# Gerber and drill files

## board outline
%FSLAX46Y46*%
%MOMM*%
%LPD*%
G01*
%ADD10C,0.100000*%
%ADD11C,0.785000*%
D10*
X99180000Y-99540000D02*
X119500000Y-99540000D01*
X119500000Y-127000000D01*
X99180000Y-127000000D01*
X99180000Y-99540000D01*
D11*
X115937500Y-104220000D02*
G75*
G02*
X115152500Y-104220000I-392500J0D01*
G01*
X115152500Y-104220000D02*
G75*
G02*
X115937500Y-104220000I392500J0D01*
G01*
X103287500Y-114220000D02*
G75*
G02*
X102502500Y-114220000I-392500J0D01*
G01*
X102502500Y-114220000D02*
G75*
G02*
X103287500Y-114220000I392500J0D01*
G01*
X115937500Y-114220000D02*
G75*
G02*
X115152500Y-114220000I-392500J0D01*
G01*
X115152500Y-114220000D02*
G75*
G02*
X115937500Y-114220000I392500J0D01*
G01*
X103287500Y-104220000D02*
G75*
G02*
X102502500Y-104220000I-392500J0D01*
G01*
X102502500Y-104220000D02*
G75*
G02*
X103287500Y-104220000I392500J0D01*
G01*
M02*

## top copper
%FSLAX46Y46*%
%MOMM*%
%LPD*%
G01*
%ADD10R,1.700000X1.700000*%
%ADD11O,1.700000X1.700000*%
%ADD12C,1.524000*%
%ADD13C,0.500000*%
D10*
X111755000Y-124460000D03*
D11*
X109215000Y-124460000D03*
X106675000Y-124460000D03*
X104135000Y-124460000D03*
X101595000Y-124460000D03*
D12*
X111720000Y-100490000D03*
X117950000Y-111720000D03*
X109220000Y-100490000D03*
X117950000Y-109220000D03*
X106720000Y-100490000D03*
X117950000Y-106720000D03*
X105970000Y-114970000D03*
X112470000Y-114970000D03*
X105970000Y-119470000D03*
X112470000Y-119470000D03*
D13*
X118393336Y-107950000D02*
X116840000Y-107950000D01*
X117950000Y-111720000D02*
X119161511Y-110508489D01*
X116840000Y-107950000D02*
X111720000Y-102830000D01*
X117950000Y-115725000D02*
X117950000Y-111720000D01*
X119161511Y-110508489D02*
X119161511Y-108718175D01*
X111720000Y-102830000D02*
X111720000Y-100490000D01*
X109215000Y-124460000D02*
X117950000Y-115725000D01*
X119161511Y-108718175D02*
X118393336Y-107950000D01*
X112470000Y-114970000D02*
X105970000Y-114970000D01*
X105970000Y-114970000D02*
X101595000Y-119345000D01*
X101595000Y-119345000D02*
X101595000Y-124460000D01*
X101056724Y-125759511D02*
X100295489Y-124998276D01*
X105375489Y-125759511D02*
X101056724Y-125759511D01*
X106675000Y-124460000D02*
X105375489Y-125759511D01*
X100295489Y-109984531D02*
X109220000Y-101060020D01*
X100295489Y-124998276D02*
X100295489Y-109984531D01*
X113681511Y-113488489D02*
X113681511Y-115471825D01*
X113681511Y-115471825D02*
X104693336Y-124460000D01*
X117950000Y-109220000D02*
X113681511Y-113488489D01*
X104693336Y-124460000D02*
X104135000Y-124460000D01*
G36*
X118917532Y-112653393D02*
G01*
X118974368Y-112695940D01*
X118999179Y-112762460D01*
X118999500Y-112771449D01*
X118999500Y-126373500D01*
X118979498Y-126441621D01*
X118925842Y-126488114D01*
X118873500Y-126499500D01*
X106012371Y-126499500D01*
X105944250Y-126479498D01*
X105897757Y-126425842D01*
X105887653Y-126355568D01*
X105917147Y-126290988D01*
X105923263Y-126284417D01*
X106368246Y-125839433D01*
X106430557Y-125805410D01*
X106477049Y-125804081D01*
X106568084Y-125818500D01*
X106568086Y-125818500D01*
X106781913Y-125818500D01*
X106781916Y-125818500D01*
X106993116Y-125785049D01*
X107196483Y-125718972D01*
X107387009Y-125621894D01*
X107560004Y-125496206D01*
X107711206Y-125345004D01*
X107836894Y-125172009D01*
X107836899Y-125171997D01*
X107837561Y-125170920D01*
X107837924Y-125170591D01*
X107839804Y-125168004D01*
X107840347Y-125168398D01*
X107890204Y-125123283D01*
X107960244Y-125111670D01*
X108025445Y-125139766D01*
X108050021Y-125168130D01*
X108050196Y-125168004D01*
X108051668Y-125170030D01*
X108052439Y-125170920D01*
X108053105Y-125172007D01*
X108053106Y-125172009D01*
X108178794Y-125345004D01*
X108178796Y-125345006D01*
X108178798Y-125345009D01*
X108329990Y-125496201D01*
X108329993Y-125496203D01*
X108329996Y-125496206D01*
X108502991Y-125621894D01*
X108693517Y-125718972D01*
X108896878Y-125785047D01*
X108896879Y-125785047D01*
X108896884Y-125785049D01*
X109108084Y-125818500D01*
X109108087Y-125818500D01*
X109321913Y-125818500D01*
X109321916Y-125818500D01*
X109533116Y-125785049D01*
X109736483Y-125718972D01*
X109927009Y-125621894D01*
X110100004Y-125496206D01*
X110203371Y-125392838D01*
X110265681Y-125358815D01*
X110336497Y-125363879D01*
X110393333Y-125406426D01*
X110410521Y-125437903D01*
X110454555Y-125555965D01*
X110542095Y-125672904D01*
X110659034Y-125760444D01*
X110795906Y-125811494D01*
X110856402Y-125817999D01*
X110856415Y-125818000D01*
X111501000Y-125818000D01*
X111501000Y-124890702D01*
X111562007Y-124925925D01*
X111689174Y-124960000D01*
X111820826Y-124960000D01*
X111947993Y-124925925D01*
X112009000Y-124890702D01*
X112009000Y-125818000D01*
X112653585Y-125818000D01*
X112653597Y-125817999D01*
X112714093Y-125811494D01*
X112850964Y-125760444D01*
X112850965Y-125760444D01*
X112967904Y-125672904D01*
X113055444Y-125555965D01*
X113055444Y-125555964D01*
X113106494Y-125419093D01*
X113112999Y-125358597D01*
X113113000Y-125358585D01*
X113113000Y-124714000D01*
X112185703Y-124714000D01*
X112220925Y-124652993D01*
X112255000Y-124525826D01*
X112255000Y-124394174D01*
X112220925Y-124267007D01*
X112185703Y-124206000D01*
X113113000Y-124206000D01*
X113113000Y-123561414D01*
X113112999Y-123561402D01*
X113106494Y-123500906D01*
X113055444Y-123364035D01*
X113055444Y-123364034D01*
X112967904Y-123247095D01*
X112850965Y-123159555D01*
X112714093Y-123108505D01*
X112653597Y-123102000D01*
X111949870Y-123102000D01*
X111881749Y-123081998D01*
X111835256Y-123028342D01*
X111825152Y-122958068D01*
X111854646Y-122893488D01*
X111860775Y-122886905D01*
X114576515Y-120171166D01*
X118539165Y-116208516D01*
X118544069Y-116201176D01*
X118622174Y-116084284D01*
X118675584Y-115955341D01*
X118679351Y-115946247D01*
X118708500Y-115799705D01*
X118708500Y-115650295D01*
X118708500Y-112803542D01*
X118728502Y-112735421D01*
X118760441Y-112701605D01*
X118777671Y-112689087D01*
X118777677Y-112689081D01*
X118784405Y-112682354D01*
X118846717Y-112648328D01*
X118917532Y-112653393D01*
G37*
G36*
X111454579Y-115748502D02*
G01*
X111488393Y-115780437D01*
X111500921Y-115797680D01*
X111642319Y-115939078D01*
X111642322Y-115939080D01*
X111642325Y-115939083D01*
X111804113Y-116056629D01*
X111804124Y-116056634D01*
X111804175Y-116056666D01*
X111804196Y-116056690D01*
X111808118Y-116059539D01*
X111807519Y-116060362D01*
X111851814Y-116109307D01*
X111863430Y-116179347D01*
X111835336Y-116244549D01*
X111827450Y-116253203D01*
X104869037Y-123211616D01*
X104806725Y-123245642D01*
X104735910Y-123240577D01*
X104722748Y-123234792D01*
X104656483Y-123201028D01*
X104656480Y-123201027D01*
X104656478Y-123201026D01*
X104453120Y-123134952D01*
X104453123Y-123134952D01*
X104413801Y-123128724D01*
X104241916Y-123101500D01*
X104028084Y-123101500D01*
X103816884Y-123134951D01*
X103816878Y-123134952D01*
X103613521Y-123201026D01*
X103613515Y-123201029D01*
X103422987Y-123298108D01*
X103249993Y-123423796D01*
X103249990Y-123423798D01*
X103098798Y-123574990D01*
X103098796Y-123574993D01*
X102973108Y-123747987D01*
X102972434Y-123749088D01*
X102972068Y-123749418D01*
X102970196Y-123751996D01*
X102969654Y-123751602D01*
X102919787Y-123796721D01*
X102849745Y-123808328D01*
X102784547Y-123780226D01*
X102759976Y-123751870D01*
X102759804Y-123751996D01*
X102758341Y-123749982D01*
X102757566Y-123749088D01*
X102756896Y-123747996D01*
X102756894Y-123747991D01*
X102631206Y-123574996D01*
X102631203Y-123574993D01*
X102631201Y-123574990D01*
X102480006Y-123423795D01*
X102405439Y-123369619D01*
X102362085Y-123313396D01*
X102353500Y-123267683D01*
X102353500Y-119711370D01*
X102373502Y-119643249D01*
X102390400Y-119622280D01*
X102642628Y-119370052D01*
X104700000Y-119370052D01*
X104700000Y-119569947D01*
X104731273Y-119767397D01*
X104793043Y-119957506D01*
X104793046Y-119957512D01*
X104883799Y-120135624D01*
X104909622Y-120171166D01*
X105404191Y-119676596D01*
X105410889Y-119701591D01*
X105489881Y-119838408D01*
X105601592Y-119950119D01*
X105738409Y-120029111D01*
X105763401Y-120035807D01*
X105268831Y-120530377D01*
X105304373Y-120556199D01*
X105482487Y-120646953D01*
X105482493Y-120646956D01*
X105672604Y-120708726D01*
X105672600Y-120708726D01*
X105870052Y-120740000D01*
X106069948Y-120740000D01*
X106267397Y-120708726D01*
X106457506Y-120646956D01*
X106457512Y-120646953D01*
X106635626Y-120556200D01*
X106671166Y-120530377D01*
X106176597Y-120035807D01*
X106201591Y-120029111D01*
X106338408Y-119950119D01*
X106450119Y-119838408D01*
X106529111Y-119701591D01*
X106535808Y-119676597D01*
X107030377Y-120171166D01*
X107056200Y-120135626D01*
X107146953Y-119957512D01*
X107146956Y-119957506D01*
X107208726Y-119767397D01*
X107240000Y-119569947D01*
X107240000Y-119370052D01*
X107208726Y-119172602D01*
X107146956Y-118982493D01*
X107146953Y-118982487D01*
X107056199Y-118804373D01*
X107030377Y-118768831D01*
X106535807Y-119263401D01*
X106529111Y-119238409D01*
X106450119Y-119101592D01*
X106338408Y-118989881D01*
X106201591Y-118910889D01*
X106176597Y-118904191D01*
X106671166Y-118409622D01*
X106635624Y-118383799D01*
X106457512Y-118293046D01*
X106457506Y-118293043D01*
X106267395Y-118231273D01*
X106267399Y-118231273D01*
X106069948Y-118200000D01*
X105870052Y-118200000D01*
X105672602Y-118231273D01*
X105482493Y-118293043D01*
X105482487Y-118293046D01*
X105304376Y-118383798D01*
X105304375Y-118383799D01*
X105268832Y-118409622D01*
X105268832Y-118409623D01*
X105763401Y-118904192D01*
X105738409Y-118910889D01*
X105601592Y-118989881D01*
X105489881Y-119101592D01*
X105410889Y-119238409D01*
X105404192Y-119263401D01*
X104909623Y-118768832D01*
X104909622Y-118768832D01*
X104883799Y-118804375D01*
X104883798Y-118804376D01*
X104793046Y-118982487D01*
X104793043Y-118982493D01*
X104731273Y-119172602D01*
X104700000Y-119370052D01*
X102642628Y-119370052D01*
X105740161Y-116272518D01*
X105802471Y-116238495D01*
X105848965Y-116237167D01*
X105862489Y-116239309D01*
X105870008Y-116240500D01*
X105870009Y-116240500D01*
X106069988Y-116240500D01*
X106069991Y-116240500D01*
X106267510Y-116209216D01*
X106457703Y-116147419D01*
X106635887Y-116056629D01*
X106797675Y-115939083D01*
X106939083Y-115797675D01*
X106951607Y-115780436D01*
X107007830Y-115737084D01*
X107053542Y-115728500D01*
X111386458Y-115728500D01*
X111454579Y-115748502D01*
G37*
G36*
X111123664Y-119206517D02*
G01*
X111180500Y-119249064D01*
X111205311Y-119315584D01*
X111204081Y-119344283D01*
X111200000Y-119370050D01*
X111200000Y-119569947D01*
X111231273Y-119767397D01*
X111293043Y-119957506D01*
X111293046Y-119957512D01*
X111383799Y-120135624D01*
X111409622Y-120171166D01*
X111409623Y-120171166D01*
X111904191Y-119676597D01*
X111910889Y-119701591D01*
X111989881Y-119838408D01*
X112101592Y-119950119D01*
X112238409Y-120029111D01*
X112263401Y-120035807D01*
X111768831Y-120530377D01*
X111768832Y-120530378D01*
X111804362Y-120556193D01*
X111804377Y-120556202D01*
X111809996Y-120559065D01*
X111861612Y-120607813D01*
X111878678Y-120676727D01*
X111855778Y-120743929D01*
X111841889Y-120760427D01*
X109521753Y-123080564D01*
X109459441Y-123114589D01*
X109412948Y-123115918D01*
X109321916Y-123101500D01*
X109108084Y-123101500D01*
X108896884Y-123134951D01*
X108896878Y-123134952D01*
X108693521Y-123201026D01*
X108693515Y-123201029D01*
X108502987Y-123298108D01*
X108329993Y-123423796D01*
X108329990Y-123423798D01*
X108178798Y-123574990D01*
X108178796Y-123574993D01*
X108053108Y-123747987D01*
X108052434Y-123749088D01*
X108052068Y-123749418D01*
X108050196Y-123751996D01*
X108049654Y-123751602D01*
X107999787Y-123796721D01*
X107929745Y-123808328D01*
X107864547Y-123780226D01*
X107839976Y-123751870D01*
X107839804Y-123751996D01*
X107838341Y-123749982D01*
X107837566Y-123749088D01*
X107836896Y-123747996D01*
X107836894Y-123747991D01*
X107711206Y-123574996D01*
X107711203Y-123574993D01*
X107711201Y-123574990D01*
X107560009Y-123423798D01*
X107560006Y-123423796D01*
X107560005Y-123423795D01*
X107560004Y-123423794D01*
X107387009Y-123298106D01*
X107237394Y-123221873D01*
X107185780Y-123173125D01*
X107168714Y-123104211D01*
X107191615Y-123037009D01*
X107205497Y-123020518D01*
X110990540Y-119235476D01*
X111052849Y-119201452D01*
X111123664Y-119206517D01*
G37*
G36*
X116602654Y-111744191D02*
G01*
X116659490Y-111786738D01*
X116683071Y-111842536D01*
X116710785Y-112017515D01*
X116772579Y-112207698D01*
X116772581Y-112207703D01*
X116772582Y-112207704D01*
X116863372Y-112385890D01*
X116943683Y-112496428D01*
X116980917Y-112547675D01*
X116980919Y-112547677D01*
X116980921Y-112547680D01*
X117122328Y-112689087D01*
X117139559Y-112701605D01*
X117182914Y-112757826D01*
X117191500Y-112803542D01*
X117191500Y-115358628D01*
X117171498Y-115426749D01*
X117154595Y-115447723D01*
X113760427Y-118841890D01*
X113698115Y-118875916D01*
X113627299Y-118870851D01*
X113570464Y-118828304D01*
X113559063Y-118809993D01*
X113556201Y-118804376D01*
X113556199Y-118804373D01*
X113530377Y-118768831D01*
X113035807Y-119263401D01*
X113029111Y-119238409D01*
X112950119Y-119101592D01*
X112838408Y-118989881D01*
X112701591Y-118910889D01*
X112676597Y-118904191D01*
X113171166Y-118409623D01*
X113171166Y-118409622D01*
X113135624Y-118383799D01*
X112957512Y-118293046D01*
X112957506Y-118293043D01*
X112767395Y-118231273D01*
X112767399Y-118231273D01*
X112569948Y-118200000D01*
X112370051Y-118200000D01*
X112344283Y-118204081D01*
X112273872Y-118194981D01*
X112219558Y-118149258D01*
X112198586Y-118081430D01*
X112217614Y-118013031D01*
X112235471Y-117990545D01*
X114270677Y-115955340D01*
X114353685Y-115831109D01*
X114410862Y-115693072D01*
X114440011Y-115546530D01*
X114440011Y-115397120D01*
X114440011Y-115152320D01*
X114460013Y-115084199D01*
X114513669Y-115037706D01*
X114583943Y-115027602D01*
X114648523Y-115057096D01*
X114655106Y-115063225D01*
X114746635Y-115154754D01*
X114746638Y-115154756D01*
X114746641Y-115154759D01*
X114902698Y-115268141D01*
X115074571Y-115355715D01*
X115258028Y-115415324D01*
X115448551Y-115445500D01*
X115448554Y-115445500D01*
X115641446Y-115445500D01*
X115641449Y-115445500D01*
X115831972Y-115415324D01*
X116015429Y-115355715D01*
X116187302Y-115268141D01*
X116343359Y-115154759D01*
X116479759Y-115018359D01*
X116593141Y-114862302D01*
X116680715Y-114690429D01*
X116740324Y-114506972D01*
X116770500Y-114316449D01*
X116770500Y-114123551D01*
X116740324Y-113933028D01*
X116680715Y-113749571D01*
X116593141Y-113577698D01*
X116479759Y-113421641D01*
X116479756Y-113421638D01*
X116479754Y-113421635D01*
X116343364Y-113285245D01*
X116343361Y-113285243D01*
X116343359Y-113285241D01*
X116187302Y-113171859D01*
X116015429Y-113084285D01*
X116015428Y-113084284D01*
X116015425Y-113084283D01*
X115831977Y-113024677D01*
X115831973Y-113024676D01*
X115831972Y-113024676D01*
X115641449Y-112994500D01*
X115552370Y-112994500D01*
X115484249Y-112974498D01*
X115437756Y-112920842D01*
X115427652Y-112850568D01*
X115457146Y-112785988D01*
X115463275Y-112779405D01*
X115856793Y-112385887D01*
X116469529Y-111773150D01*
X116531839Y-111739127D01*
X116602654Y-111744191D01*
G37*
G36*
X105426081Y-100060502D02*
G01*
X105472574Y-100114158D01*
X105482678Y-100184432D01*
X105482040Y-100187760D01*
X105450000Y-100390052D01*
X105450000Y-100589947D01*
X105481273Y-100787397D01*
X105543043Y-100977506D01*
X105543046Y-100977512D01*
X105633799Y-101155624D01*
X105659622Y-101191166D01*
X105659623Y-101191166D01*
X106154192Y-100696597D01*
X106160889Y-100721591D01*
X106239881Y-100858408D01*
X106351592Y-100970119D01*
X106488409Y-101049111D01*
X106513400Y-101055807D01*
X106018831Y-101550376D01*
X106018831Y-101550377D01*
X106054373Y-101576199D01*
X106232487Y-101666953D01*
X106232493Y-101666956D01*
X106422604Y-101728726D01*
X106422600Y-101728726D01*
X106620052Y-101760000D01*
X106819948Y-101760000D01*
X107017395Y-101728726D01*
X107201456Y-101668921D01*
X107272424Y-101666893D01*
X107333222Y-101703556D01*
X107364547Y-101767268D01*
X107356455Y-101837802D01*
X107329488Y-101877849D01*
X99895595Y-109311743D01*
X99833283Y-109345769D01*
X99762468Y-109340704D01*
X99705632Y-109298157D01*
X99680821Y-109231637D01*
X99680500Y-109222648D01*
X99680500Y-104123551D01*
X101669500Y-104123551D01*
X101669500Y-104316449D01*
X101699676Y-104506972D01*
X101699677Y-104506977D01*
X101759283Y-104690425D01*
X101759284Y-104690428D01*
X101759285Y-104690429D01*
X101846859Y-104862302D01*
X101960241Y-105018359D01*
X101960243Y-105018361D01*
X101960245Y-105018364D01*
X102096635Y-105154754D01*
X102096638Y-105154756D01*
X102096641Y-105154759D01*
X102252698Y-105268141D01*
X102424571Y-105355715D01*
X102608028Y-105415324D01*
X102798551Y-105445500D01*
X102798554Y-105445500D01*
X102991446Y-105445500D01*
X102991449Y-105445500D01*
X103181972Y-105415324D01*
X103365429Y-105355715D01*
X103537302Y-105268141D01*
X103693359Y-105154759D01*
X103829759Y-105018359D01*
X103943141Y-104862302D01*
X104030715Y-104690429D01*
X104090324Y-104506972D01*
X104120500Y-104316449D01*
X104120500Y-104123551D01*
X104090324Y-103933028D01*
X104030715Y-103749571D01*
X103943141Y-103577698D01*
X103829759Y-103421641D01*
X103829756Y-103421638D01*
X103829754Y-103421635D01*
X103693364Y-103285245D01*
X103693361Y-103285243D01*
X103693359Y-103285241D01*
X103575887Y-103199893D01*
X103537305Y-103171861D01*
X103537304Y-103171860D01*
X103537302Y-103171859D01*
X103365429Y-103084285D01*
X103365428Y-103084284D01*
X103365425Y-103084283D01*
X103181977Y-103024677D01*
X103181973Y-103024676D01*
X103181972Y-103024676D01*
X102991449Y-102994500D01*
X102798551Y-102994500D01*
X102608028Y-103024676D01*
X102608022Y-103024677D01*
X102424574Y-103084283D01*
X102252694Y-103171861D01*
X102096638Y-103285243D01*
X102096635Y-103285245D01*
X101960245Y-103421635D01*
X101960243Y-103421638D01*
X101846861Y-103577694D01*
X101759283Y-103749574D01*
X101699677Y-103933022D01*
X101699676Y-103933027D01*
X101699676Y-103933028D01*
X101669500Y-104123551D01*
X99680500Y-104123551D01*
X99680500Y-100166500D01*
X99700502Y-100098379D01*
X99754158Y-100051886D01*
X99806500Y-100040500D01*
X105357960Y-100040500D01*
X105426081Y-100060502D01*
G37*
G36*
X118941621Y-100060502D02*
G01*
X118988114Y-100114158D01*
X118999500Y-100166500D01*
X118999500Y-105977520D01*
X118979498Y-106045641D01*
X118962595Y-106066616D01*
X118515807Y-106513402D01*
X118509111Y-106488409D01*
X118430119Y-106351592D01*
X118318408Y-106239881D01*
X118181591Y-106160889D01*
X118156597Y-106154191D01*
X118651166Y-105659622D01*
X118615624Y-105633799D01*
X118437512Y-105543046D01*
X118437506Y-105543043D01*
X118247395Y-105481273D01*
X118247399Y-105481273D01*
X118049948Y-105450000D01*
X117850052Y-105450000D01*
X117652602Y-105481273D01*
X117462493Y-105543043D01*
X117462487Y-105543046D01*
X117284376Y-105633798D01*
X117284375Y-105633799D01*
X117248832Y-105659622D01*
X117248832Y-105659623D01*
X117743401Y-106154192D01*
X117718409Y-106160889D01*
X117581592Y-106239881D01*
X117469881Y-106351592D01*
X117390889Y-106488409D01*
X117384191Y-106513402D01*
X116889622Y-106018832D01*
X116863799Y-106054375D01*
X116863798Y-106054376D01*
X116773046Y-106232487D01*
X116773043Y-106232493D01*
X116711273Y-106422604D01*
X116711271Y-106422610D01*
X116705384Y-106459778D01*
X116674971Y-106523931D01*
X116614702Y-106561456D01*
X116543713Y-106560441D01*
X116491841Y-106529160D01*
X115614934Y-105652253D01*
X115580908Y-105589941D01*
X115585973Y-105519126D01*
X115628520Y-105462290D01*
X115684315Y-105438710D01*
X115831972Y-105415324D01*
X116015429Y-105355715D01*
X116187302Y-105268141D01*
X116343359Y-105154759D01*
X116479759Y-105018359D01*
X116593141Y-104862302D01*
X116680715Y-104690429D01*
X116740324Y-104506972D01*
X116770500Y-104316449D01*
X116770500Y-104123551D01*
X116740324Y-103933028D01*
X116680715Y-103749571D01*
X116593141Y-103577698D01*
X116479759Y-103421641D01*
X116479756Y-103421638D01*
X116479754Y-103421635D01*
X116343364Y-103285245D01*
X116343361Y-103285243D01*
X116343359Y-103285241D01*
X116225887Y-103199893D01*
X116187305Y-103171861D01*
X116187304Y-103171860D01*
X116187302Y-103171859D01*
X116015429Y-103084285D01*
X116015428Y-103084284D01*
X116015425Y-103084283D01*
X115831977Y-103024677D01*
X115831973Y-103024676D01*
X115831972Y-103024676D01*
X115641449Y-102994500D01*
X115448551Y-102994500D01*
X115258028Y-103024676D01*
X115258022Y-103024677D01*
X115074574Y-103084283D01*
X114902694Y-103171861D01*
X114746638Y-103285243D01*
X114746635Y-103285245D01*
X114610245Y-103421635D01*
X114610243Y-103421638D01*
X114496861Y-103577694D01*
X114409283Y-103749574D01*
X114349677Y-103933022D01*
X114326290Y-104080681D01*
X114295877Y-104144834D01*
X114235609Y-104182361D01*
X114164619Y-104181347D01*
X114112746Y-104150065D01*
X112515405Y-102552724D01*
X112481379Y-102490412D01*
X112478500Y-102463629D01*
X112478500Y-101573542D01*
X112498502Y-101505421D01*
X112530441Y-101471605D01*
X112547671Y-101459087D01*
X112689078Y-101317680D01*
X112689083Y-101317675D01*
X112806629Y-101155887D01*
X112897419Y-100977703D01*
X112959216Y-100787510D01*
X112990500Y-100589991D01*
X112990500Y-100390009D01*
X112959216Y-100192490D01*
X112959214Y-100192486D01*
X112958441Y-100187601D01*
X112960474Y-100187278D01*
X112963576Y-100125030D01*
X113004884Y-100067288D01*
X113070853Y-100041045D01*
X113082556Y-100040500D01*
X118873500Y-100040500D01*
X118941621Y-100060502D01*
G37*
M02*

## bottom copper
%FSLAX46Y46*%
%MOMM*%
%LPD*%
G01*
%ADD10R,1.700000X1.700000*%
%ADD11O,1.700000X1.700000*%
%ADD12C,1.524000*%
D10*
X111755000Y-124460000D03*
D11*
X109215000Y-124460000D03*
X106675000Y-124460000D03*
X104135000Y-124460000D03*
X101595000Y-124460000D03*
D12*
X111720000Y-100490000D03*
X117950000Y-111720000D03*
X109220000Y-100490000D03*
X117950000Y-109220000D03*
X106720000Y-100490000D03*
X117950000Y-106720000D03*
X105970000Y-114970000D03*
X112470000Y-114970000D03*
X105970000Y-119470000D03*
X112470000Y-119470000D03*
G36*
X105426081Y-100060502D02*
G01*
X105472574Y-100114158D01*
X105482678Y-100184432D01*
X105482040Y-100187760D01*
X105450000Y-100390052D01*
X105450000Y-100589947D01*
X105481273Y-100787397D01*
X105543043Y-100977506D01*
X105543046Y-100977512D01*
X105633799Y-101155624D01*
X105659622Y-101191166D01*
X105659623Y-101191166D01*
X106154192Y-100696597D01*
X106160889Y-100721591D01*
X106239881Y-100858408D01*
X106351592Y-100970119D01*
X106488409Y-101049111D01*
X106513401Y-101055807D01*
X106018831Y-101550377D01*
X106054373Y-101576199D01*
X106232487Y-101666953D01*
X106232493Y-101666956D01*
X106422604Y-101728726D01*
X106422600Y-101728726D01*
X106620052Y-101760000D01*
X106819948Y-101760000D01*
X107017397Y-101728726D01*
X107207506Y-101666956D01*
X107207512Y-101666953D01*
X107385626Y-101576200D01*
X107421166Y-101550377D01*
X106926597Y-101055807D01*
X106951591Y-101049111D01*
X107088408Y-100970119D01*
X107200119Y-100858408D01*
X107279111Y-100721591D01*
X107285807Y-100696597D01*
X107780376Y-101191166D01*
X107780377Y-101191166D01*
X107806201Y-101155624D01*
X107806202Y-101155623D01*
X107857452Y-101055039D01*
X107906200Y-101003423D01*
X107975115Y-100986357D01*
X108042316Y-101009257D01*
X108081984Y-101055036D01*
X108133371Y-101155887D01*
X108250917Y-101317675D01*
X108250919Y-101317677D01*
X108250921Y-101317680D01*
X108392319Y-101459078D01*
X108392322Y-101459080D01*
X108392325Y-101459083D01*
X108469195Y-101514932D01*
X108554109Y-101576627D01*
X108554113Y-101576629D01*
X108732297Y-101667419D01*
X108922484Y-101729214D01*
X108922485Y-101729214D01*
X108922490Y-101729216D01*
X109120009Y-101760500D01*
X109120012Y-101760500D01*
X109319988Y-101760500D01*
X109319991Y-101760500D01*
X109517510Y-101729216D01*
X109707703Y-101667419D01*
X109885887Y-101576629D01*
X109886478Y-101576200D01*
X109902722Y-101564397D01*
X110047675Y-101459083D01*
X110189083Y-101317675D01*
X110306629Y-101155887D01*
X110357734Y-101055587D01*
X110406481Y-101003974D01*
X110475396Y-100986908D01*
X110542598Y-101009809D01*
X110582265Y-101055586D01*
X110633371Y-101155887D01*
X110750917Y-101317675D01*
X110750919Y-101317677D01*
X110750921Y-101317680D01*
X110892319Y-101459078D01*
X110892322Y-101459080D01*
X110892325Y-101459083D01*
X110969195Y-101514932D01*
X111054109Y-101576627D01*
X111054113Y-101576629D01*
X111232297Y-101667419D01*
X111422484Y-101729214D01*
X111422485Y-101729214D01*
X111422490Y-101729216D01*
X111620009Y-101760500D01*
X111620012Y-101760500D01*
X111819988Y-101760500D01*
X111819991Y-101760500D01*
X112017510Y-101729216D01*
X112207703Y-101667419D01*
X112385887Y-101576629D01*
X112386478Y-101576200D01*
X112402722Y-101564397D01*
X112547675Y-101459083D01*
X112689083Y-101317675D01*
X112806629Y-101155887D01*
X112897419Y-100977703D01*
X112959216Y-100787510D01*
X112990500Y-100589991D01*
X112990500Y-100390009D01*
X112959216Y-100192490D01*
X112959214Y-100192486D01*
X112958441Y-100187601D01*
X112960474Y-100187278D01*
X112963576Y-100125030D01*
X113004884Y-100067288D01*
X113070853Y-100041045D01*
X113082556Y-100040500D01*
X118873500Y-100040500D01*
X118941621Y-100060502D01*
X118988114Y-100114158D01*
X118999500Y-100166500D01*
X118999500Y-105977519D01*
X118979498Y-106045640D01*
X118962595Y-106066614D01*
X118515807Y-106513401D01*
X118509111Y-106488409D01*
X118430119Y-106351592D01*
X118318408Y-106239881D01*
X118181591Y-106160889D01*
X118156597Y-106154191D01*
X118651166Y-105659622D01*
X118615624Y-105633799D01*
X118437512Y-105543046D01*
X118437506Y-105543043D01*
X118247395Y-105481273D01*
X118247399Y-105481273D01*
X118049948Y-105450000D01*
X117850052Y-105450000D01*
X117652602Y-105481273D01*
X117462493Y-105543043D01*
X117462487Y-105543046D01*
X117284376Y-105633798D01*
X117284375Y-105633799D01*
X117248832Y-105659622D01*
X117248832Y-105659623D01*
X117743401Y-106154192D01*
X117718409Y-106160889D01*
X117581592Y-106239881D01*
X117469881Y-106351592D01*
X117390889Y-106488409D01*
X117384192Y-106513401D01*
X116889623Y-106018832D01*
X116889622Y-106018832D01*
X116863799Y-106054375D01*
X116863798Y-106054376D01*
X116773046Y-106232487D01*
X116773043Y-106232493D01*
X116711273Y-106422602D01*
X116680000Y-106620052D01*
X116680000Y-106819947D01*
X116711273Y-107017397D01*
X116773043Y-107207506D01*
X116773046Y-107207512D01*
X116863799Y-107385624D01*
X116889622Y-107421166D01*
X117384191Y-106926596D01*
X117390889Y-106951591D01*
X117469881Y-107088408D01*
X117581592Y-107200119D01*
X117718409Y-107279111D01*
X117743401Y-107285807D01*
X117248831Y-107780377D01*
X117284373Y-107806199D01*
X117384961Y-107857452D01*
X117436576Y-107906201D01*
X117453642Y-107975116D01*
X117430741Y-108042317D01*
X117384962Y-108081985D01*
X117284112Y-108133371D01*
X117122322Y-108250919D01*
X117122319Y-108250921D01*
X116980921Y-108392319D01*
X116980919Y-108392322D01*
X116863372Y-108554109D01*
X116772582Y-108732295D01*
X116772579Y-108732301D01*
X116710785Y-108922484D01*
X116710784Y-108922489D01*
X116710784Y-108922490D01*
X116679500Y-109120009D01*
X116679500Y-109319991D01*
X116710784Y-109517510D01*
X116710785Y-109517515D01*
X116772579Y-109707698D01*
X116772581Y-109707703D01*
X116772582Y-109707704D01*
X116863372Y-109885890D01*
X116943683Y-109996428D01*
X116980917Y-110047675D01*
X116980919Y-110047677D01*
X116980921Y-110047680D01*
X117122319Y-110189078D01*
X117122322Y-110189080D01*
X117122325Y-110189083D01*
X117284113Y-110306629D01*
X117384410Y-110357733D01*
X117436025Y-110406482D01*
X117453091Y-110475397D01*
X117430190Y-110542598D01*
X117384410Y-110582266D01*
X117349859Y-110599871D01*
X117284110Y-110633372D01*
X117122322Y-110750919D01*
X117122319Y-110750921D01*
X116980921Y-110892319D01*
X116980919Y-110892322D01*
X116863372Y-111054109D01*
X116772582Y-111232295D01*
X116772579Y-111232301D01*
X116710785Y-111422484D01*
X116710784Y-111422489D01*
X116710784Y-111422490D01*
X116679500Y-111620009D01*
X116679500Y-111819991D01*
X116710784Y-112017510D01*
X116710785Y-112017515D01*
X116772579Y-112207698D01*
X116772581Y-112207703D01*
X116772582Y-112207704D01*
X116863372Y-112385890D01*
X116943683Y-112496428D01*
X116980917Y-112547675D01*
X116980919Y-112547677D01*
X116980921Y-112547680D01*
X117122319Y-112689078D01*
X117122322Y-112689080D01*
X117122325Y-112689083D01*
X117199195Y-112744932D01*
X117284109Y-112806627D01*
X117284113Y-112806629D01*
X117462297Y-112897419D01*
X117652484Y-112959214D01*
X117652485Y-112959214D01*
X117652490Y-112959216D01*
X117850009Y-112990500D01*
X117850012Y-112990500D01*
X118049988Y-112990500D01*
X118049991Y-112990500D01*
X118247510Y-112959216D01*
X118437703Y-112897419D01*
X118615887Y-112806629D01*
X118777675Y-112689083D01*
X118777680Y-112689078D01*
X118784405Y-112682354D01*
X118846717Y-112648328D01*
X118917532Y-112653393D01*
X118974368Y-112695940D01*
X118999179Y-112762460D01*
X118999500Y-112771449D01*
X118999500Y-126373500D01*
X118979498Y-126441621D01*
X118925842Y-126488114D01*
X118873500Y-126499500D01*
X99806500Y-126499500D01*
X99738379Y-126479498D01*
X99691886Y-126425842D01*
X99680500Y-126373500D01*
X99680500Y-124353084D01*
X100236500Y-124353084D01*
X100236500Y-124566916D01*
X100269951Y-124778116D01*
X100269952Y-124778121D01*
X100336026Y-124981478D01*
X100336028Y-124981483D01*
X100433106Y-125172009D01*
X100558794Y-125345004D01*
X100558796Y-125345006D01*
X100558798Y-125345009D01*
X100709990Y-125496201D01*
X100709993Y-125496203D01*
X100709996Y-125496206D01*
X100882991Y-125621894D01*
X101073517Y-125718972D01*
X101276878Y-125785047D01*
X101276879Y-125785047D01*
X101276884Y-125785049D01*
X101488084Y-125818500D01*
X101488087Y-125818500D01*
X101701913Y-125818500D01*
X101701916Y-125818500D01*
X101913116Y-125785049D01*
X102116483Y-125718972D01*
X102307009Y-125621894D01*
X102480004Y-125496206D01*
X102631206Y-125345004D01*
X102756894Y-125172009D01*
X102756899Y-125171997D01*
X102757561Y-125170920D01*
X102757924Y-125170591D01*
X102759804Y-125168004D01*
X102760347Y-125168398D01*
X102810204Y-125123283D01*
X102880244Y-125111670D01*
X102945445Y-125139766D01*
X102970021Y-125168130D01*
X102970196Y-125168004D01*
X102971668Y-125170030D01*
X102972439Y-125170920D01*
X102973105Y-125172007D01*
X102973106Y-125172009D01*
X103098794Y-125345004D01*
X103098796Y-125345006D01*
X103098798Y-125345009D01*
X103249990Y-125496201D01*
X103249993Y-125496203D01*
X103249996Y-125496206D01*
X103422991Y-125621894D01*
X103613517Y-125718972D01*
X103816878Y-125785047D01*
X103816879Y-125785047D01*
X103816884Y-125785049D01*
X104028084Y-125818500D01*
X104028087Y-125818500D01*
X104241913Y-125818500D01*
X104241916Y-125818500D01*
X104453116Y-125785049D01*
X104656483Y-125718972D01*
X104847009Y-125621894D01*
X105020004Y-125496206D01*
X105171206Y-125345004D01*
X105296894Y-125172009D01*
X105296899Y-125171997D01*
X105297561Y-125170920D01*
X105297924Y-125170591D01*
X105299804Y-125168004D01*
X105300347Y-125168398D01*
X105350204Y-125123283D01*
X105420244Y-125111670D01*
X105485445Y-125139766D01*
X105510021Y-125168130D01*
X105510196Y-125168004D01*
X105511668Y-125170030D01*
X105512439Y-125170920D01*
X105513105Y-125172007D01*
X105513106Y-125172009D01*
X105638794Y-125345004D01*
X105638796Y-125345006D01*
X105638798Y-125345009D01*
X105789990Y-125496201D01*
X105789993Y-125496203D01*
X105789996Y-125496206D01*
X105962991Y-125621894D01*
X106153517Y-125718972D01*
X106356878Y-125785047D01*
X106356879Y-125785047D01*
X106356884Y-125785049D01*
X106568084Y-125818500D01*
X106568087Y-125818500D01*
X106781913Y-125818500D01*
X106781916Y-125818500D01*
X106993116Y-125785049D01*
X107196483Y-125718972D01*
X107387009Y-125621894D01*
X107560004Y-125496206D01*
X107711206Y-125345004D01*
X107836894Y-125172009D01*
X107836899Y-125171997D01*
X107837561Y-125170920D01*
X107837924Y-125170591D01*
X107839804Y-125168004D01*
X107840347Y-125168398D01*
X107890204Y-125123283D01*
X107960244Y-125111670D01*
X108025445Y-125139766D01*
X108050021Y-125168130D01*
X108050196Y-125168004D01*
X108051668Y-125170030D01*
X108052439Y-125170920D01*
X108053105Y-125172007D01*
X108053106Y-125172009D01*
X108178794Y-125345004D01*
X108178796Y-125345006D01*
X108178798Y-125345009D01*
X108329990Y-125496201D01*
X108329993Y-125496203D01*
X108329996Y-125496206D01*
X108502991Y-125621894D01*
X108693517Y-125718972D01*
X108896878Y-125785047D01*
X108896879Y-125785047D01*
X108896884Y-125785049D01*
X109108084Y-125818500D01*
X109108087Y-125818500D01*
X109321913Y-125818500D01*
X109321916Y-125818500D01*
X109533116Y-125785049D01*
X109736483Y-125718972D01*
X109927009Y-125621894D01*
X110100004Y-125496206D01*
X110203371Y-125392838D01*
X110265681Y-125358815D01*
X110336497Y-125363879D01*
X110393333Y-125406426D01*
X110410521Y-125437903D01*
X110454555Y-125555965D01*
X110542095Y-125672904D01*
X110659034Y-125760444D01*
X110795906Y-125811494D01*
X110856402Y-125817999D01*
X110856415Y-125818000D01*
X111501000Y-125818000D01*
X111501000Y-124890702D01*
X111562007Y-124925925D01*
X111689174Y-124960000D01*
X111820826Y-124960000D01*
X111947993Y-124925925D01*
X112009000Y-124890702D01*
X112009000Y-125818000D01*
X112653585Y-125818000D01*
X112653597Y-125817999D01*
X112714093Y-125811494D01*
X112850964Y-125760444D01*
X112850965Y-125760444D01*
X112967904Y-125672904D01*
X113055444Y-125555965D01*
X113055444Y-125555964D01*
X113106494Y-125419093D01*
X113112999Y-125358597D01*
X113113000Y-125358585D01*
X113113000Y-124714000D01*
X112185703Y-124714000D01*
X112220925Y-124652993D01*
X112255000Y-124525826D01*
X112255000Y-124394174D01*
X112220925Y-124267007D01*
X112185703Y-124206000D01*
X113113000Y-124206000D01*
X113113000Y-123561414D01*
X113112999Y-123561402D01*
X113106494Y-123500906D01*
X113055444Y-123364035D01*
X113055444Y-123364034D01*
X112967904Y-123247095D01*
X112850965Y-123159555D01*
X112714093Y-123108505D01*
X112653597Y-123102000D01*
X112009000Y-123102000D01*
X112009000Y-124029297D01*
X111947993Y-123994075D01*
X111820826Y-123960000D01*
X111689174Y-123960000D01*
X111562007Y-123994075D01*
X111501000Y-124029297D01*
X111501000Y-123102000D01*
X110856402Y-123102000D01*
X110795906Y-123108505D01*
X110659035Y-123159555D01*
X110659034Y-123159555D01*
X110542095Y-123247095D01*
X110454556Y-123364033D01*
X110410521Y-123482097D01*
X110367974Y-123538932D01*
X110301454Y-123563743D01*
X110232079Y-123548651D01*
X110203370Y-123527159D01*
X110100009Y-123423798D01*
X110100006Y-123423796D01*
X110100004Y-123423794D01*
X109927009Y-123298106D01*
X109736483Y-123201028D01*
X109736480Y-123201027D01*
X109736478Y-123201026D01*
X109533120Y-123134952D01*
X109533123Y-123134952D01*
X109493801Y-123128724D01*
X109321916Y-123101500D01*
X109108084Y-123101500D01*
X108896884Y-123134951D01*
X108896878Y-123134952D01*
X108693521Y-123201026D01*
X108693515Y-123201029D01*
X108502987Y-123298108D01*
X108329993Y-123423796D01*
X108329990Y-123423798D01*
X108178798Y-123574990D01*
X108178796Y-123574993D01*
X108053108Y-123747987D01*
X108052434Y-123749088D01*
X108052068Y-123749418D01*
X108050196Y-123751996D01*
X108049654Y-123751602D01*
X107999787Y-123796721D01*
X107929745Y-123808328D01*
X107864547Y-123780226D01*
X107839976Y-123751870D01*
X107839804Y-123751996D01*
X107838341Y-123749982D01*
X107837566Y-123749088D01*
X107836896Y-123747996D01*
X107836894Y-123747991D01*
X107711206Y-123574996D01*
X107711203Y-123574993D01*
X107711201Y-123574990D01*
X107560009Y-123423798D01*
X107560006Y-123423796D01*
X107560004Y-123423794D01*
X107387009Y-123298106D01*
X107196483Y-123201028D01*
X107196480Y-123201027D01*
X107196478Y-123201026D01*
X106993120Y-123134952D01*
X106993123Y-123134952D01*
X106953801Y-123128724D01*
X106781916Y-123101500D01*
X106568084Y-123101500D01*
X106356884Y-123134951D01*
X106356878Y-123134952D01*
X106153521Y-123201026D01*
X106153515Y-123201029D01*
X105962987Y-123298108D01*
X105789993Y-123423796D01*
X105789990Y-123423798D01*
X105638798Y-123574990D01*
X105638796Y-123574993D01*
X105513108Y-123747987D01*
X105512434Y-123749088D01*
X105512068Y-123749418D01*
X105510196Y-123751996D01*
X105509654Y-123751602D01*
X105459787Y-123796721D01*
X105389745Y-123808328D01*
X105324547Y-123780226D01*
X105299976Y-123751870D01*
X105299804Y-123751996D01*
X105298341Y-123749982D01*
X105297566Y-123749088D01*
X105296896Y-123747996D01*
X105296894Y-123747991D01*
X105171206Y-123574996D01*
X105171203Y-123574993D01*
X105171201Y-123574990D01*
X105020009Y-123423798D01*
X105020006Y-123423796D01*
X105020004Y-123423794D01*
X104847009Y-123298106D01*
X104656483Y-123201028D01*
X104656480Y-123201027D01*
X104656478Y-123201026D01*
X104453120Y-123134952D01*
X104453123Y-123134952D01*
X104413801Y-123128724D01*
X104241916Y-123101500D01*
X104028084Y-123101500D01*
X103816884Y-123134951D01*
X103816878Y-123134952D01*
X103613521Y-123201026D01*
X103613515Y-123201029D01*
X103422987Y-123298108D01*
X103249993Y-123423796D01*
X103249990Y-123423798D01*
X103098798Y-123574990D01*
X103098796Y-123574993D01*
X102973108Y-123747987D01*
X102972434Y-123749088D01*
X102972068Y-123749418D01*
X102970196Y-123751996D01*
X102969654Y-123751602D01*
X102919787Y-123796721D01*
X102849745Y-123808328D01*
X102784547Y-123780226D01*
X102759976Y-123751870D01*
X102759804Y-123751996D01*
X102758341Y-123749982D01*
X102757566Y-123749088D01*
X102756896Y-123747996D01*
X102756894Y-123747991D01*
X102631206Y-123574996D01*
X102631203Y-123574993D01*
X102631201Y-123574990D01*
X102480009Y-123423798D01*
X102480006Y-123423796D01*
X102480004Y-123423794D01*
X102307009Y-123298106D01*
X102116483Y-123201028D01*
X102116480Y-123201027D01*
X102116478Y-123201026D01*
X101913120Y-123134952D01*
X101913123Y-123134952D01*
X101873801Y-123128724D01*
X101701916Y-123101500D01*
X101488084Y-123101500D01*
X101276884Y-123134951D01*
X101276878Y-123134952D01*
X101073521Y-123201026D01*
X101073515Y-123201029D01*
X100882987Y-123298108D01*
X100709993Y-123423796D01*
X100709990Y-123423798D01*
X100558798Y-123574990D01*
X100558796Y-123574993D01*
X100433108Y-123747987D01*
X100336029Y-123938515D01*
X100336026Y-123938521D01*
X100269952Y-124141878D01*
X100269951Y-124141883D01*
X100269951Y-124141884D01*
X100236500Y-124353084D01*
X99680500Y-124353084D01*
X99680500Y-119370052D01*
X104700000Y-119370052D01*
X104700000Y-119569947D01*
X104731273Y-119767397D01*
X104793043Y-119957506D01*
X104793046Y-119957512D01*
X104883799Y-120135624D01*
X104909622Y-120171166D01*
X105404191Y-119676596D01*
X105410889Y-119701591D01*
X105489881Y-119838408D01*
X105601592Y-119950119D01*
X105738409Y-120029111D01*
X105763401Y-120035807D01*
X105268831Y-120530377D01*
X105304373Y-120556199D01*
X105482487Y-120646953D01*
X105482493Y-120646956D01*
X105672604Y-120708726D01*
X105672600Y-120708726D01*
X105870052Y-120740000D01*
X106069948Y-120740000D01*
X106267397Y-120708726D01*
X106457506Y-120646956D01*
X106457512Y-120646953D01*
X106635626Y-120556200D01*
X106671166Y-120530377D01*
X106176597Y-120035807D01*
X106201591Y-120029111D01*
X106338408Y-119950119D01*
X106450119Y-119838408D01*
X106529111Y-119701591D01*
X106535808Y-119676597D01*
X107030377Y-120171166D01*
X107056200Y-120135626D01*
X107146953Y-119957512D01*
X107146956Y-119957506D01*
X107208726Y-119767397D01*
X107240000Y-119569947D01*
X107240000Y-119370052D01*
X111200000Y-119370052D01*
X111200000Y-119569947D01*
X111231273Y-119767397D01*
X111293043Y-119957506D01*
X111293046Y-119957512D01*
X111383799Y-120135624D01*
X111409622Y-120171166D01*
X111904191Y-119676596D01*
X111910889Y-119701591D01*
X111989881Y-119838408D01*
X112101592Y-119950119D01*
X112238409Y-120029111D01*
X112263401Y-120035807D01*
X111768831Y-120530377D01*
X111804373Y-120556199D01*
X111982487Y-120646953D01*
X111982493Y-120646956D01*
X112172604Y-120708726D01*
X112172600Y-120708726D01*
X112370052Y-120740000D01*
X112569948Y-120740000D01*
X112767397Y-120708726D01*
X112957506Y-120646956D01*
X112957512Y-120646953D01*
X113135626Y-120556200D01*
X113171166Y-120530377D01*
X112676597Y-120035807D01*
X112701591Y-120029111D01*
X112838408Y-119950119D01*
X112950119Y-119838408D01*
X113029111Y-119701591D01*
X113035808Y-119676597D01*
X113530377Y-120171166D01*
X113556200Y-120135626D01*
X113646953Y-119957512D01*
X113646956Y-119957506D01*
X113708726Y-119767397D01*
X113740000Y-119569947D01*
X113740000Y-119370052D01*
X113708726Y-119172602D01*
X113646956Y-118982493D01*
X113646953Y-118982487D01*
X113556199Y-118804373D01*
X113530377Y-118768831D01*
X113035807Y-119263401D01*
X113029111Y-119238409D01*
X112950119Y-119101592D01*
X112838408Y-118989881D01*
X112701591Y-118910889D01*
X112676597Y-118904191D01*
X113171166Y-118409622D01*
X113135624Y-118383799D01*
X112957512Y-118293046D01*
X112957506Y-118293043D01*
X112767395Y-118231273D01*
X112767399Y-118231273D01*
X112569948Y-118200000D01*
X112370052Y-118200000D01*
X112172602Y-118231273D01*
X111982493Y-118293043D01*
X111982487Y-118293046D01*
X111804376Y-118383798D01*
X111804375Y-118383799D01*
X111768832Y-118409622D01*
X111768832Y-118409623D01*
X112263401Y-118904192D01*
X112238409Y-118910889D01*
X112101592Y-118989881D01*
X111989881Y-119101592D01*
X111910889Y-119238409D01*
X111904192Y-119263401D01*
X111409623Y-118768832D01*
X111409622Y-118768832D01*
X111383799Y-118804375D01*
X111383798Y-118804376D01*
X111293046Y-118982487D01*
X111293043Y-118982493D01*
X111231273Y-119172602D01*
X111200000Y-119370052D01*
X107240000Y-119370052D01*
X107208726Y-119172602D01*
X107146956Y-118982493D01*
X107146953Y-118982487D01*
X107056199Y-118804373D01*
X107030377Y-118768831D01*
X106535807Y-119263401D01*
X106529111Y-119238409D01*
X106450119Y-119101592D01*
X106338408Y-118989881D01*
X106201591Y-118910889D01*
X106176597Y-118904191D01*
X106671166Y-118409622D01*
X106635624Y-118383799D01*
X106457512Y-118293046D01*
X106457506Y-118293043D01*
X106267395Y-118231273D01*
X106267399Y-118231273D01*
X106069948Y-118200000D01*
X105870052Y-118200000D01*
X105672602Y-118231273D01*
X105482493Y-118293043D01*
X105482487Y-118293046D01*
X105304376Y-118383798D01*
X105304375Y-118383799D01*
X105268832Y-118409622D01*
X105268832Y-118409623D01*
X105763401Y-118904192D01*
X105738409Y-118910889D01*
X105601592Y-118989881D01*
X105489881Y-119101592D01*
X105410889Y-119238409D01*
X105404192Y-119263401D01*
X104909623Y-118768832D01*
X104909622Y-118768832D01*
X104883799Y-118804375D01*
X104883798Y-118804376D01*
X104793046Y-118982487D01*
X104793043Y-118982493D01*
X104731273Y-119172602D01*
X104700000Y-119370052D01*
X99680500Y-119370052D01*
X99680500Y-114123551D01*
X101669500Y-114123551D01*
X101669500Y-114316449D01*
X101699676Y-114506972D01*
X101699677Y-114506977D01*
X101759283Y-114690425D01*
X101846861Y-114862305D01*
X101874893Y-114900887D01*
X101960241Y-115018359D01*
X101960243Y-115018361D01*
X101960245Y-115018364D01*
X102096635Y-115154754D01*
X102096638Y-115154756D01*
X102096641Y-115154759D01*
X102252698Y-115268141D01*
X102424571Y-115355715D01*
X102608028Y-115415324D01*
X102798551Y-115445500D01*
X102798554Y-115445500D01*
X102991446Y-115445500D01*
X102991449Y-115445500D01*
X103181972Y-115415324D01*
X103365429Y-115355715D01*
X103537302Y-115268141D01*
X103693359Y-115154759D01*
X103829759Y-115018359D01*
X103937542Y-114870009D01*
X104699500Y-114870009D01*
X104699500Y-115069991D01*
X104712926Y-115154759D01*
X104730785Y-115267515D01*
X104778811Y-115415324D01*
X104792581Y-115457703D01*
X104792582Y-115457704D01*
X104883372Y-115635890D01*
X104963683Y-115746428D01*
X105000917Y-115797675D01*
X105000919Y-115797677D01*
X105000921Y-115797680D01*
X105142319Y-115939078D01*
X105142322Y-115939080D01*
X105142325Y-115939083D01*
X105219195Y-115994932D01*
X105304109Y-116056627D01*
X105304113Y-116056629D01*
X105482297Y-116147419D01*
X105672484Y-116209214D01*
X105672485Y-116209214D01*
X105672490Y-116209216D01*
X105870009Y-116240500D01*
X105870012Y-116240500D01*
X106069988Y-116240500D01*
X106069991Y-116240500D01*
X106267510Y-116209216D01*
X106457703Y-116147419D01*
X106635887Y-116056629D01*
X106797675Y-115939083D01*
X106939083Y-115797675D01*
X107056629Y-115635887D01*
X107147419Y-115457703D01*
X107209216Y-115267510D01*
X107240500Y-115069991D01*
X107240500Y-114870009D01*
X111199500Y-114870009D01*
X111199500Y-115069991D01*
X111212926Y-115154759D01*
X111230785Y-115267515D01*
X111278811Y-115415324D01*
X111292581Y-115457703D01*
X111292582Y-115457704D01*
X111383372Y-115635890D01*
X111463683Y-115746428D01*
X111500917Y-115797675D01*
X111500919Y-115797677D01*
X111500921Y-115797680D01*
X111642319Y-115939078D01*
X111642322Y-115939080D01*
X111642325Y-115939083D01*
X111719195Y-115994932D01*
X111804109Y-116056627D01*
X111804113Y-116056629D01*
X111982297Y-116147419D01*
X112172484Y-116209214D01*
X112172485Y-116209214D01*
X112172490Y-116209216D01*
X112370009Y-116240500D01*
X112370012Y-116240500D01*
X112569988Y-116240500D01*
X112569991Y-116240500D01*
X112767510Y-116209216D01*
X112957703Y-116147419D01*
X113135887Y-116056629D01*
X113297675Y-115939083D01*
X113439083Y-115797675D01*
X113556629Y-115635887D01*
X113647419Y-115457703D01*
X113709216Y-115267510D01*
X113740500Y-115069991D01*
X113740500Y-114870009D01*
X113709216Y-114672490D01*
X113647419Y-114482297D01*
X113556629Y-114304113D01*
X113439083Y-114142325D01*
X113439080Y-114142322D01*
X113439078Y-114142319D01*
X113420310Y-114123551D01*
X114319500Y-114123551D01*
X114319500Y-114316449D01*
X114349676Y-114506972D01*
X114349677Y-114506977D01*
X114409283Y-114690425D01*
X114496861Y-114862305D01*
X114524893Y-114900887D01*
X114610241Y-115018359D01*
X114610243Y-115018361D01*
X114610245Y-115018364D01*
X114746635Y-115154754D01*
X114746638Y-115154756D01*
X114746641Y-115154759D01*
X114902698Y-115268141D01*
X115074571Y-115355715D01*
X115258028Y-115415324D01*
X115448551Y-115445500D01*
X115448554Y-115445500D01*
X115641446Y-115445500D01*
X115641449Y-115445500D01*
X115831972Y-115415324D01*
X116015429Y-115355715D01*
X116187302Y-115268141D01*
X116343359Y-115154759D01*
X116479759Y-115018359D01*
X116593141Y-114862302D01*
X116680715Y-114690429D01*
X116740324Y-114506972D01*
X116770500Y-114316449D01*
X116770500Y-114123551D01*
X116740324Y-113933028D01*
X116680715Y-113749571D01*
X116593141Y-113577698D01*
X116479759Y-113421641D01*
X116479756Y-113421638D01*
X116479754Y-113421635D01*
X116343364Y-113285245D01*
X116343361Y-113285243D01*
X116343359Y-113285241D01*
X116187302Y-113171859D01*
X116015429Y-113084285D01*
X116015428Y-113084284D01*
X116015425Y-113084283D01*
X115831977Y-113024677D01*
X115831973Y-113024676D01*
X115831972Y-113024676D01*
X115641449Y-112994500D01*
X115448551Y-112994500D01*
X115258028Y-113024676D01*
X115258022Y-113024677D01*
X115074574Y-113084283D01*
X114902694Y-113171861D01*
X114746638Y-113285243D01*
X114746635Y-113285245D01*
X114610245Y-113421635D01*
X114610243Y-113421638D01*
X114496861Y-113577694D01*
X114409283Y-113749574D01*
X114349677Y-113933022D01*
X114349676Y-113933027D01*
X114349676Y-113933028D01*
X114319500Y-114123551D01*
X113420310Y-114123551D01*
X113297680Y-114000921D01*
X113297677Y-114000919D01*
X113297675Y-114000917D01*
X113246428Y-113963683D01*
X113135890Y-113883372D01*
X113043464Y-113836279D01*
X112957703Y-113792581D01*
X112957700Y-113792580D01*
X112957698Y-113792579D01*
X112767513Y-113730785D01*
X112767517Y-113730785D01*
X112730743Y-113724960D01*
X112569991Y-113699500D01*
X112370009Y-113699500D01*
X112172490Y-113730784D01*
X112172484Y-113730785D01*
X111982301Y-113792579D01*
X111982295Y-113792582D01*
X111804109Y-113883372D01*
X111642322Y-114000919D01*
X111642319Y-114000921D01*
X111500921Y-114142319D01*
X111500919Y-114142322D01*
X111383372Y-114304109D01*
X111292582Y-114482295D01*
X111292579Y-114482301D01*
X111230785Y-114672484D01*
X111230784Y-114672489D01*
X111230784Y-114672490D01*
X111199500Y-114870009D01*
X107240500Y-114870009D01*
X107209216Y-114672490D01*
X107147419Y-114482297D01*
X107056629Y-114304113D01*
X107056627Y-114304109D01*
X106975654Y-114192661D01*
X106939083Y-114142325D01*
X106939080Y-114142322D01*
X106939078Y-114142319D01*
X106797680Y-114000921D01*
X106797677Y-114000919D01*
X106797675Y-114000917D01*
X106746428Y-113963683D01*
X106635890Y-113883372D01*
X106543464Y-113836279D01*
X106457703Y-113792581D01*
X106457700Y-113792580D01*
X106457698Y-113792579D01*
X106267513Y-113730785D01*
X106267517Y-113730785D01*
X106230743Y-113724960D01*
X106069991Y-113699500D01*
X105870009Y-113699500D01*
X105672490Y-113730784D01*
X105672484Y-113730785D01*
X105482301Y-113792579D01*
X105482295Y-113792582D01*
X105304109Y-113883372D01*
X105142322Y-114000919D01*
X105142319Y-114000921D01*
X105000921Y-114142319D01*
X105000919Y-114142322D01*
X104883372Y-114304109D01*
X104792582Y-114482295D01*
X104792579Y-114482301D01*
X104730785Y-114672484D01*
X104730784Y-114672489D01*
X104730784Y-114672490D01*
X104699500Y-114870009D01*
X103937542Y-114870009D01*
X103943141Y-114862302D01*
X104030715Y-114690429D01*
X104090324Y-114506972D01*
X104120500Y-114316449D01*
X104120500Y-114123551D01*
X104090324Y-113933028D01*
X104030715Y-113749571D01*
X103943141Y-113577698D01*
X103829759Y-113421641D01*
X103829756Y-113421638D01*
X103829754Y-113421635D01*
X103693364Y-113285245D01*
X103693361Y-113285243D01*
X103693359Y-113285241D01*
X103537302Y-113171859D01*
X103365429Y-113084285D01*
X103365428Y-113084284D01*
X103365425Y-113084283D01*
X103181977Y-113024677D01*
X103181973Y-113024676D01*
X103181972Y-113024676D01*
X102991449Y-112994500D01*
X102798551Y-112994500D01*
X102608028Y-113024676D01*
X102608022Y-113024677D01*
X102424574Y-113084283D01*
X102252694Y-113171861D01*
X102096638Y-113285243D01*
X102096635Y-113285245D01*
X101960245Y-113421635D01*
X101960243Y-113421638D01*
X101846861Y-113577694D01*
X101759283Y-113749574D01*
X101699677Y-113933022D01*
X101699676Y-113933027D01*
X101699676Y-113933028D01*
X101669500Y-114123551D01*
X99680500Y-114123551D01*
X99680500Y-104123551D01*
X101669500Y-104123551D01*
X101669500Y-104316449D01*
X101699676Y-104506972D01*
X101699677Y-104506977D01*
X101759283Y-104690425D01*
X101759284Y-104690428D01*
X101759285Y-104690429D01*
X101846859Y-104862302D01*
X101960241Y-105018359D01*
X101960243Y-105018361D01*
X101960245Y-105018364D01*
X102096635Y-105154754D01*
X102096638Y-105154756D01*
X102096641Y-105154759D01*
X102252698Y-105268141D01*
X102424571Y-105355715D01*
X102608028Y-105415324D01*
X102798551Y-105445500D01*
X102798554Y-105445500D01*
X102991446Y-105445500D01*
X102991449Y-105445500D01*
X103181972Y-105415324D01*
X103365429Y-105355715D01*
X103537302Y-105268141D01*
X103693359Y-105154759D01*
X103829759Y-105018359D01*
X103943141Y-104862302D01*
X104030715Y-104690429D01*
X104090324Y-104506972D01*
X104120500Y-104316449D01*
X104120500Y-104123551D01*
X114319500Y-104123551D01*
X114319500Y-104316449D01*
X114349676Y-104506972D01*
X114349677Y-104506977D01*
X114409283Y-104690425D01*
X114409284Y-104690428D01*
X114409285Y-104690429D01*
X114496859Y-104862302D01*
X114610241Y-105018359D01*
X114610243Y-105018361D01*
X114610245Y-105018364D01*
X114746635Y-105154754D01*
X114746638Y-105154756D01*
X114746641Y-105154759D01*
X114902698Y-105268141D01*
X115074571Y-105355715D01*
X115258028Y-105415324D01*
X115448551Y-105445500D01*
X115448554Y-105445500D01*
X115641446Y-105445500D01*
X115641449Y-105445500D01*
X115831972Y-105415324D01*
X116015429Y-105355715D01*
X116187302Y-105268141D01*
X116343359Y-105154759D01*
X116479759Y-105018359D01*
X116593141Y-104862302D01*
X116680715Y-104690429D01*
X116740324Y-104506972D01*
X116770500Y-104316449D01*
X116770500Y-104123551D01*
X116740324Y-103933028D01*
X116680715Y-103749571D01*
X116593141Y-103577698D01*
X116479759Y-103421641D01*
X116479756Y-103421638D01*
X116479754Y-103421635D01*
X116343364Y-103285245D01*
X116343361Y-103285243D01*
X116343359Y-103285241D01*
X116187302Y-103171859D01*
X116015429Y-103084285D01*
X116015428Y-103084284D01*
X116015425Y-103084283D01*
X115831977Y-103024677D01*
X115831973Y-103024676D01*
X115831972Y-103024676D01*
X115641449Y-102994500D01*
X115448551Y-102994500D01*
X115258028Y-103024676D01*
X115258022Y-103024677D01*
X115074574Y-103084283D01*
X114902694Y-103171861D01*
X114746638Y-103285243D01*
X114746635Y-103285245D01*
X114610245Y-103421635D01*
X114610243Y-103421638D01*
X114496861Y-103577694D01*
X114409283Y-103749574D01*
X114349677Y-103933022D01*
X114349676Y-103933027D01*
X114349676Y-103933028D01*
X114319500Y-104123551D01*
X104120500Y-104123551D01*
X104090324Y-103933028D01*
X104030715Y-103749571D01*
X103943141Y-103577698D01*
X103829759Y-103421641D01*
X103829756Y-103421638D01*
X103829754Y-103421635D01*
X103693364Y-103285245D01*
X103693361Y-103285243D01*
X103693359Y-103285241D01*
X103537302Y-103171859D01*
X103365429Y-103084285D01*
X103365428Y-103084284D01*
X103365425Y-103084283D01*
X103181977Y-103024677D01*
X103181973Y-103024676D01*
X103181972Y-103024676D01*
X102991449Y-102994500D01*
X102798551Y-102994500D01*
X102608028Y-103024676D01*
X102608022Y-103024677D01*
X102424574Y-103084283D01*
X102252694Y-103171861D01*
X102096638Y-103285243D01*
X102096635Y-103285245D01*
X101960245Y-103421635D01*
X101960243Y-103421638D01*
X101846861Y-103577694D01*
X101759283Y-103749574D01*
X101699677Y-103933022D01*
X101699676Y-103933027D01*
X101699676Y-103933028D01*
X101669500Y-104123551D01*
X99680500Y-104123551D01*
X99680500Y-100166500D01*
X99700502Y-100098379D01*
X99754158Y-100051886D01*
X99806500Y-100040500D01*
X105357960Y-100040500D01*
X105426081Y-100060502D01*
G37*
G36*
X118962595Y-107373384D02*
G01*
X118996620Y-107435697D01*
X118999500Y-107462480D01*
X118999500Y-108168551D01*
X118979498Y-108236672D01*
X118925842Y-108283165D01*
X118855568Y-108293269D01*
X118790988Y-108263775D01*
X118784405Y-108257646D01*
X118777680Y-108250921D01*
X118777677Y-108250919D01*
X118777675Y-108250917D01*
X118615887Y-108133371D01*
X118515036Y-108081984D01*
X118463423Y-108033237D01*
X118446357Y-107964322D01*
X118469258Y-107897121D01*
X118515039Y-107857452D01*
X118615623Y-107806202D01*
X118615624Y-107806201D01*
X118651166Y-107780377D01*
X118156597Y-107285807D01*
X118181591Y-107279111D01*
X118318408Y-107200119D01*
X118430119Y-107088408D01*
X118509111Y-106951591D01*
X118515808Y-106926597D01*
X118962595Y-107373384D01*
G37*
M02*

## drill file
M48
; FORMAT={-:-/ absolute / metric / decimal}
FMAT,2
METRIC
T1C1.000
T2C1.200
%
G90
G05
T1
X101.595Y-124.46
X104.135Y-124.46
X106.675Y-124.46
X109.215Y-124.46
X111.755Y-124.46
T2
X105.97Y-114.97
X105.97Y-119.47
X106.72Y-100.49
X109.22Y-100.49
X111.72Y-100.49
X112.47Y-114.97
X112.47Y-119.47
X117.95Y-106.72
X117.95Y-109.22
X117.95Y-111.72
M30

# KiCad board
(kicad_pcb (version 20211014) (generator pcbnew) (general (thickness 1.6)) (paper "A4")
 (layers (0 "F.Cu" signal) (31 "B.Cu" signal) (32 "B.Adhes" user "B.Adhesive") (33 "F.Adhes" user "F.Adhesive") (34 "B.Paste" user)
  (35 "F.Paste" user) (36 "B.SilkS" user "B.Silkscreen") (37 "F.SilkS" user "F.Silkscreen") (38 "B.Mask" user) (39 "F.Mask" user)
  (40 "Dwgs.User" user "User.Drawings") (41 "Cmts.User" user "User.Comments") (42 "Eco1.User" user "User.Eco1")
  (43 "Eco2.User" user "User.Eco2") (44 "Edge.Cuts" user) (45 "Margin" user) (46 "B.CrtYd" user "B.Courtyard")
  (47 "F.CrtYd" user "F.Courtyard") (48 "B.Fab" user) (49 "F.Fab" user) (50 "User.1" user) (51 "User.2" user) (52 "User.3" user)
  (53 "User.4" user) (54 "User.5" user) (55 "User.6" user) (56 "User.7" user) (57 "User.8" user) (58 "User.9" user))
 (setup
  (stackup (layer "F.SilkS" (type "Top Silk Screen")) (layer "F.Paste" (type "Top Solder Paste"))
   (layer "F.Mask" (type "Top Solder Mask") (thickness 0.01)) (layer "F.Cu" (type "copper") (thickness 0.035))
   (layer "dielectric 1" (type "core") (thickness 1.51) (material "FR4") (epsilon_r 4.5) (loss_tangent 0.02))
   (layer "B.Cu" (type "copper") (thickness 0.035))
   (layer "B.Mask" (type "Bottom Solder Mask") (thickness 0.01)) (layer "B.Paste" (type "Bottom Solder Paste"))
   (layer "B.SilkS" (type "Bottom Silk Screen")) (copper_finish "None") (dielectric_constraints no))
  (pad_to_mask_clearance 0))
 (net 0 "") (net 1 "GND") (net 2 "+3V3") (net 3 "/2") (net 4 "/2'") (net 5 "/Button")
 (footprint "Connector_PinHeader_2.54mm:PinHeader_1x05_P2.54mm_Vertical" (layer "F.Cu") (at 111.755 124.46 -90)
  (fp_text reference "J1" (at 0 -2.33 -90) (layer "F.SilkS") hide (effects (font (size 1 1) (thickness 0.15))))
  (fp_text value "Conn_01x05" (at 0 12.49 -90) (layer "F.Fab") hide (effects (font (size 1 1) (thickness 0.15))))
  (pad "1" thru_hole rect (at 0 0 270) (size 1.7 1.7) (drill 1) (layers *.Cu *.Mask) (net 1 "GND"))
  (pad "2" thru_hole oval (at 0 2.54 270) (size 1.7 1.7) (drill 1) (layers *.Cu *.Mask) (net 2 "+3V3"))
  (pad "3" thru_hole oval (at 0 5.08 270) (size 1.7 1.7) (drill 1) (layers *.Cu *.Mask) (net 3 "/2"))
  (pad "4" thru_hole oval (at 0 7.62 270) (size 1.7 1.7) (drill 1) (layers *.Cu *.Mask) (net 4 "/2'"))
  (pad "5" thru_hole oval (at 0 10.16 270) (size 1.7 1.7) (drill 1) (layers *.Cu *.Mask) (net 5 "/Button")))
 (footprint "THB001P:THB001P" (layer "F.Cu") (at 109.22 109.22)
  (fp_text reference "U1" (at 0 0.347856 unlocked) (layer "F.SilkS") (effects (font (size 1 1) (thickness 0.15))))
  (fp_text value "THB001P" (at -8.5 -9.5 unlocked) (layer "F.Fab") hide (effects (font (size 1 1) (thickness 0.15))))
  (fp_circle (center 6.325 -5) (end 7.05 -5) (layer "Edge.Cuts") (width 0.12) (fill solid))
  (fp_circle (center -6.325 5) (end -5.6 5) (layer "Edge.Cuts") (width 0.12) (fill solid))
  (fp_circle (center 6.325 5) (end 7.05 5) (layer "Edge.Cuts") (width 0.12) (fill solid))
  (fp_circle (center -6.325 -5) (end -5.6 -5) (layer "Edge.Cuts") (width 0.12) (fill solid))
  (pad "1" thru_hole circle (at 2.5 -8.73) (size 1.524 1.524) (drill 1.2) (layers *.Cu *.Mask) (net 2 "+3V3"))
  (pad "1'" thru_hole circle (at 8.73 2.5) (size 1.524 1.524) (drill 1.2) (layers *.Cu *.Mask) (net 2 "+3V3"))
  (pad "2" thru_hole circle (at 0 -8.73) (size 1.524 1.524) (drill 1.2) (layers *.Cu *.Mask) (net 3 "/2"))
  (pad "2'" thru_hole circle (at 8.73 0) (size 1.524 1.524) (drill 1.2) (layers *.Cu *.Mask) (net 4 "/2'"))
  (pad "3" thru_hole circle (at -2.5 -8.73) (size 1.524 1.524) (drill 1.2) (layers *.Cu *.Mask) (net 1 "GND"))
  (pad "3'" thru_hole circle (at 8.73 -2.5) (size 1.524 1.524) (drill 1.2) (layers *.Cu *.Mask) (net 1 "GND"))
  (pad "a" thru_hole circle (at -3.25 5.75) (size 1.524 1.524) (drill 1.2) (layers *.Cu *.Mask) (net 5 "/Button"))
  (pad "b" thru_hole circle (at 3.25 5.75) (size 1.524 1.524) (drill 1.2) (layers *.Cu *.Mask) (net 5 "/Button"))
  (pad "c" thru_hole circle (at -3.25 10.25) (size 1.524 1.524) (drill 1.2) (layers *.Cu *.Mask) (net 1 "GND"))
  (pad "d" thru_hole circle (at 3.25 10.25) (size 1.524 1.524) (drill 1.2) (layers *.Cu *.Mask) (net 1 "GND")))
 (gr_rect (start 99.18 99.54) (end 119.5 127) (layer "Edge.Cuts") (width 0.1) (fill none))
 (segment (start 118.393336 107.95) (end 116.84 107.95) (width 0.5) (layer "F.Cu") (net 2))
 (segment (start 117.95 111.72) (end 119.161511 110.508489) (width 0.5) (layer "F.Cu") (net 2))
 (segment (start 116.84 107.95) (end 111.72 102.83) (width 0.5) (layer "F.Cu") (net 2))
 (segment (start 117.95 115.725) (end 117.95 111.72) (width 0.5) (layer "F.Cu") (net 2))
 (segment (start 119.161511 110.508489) (end 119.161511 108.718175) (width 0.5) (layer "F.Cu") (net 2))
 (segment (start 111.72 102.83) (end 111.72 100.49) (width 0.5) (layer "F.Cu") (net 2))
 (segment (start 109.215 124.46) (end 117.95 115.725) (width 0.5) (layer "F.Cu") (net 2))
 (segment (start 119.161511 108.718175) (end 118.393336 107.95) (width 0.5) (layer "F.Cu") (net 2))
 (segment (start 112.47 114.97) (end 105.97 114.97) (width 0.5) (layer "F.Cu") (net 5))
 (segment (start 105.97 114.97) (end 101.595 119.345) (width 0.5) (layer "F.Cu") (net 5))
 (segment (start 101.595 119.345) (end 101.595 124.46) (width 0.5) (layer "F.Cu") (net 5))
 (segment (start 101.056724 125.759511) (end 100.295489 124.998276) (width 0.5) (layer "F.Cu") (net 3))
 (segment (start 105.375489 125.759511) (end 101.056724 125.759511) (width 0.5) (layer "F.Cu") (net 3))
 (segment (start 106.675 124.46) (end 105.375489 125.759511) (width 0.5) (layer "F.Cu") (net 3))
 (segment (start 100.295489 109.984531) (end 109.22 101.06002) (width 0.5) (layer "F.Cu") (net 3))
 (segment (start 100.295489 124.998276) (end 100.295489 109.984531) (width 0.5) (layer "F.Cu") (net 3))
 (segment (start 113.681511 113.488489) (end 113.681511 115.471825) (width 0.5) (layer "F.Cu") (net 4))
 (segment (start 113.681511 115.471825) (end 104.693336 124.46) (width 0.5) (layer "F.Cu") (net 4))
 (segment (start 117.95 109.22) (end 113.681511 113.488489) (width 0.5) (layer "F.Cu") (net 4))
 (segment (start 104.693336 124.46) (end 104.135 124.46) (width 0.5) (layer "F.Cu") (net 4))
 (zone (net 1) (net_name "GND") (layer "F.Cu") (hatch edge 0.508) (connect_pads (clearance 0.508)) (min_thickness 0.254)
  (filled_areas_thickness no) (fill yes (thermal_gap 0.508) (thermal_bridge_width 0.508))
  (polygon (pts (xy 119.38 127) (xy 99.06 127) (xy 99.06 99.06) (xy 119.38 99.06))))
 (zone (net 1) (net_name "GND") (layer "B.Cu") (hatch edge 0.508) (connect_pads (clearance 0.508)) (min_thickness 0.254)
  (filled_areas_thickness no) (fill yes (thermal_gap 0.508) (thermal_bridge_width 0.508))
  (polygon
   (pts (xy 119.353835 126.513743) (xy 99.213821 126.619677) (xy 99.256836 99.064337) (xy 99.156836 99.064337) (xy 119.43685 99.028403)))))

